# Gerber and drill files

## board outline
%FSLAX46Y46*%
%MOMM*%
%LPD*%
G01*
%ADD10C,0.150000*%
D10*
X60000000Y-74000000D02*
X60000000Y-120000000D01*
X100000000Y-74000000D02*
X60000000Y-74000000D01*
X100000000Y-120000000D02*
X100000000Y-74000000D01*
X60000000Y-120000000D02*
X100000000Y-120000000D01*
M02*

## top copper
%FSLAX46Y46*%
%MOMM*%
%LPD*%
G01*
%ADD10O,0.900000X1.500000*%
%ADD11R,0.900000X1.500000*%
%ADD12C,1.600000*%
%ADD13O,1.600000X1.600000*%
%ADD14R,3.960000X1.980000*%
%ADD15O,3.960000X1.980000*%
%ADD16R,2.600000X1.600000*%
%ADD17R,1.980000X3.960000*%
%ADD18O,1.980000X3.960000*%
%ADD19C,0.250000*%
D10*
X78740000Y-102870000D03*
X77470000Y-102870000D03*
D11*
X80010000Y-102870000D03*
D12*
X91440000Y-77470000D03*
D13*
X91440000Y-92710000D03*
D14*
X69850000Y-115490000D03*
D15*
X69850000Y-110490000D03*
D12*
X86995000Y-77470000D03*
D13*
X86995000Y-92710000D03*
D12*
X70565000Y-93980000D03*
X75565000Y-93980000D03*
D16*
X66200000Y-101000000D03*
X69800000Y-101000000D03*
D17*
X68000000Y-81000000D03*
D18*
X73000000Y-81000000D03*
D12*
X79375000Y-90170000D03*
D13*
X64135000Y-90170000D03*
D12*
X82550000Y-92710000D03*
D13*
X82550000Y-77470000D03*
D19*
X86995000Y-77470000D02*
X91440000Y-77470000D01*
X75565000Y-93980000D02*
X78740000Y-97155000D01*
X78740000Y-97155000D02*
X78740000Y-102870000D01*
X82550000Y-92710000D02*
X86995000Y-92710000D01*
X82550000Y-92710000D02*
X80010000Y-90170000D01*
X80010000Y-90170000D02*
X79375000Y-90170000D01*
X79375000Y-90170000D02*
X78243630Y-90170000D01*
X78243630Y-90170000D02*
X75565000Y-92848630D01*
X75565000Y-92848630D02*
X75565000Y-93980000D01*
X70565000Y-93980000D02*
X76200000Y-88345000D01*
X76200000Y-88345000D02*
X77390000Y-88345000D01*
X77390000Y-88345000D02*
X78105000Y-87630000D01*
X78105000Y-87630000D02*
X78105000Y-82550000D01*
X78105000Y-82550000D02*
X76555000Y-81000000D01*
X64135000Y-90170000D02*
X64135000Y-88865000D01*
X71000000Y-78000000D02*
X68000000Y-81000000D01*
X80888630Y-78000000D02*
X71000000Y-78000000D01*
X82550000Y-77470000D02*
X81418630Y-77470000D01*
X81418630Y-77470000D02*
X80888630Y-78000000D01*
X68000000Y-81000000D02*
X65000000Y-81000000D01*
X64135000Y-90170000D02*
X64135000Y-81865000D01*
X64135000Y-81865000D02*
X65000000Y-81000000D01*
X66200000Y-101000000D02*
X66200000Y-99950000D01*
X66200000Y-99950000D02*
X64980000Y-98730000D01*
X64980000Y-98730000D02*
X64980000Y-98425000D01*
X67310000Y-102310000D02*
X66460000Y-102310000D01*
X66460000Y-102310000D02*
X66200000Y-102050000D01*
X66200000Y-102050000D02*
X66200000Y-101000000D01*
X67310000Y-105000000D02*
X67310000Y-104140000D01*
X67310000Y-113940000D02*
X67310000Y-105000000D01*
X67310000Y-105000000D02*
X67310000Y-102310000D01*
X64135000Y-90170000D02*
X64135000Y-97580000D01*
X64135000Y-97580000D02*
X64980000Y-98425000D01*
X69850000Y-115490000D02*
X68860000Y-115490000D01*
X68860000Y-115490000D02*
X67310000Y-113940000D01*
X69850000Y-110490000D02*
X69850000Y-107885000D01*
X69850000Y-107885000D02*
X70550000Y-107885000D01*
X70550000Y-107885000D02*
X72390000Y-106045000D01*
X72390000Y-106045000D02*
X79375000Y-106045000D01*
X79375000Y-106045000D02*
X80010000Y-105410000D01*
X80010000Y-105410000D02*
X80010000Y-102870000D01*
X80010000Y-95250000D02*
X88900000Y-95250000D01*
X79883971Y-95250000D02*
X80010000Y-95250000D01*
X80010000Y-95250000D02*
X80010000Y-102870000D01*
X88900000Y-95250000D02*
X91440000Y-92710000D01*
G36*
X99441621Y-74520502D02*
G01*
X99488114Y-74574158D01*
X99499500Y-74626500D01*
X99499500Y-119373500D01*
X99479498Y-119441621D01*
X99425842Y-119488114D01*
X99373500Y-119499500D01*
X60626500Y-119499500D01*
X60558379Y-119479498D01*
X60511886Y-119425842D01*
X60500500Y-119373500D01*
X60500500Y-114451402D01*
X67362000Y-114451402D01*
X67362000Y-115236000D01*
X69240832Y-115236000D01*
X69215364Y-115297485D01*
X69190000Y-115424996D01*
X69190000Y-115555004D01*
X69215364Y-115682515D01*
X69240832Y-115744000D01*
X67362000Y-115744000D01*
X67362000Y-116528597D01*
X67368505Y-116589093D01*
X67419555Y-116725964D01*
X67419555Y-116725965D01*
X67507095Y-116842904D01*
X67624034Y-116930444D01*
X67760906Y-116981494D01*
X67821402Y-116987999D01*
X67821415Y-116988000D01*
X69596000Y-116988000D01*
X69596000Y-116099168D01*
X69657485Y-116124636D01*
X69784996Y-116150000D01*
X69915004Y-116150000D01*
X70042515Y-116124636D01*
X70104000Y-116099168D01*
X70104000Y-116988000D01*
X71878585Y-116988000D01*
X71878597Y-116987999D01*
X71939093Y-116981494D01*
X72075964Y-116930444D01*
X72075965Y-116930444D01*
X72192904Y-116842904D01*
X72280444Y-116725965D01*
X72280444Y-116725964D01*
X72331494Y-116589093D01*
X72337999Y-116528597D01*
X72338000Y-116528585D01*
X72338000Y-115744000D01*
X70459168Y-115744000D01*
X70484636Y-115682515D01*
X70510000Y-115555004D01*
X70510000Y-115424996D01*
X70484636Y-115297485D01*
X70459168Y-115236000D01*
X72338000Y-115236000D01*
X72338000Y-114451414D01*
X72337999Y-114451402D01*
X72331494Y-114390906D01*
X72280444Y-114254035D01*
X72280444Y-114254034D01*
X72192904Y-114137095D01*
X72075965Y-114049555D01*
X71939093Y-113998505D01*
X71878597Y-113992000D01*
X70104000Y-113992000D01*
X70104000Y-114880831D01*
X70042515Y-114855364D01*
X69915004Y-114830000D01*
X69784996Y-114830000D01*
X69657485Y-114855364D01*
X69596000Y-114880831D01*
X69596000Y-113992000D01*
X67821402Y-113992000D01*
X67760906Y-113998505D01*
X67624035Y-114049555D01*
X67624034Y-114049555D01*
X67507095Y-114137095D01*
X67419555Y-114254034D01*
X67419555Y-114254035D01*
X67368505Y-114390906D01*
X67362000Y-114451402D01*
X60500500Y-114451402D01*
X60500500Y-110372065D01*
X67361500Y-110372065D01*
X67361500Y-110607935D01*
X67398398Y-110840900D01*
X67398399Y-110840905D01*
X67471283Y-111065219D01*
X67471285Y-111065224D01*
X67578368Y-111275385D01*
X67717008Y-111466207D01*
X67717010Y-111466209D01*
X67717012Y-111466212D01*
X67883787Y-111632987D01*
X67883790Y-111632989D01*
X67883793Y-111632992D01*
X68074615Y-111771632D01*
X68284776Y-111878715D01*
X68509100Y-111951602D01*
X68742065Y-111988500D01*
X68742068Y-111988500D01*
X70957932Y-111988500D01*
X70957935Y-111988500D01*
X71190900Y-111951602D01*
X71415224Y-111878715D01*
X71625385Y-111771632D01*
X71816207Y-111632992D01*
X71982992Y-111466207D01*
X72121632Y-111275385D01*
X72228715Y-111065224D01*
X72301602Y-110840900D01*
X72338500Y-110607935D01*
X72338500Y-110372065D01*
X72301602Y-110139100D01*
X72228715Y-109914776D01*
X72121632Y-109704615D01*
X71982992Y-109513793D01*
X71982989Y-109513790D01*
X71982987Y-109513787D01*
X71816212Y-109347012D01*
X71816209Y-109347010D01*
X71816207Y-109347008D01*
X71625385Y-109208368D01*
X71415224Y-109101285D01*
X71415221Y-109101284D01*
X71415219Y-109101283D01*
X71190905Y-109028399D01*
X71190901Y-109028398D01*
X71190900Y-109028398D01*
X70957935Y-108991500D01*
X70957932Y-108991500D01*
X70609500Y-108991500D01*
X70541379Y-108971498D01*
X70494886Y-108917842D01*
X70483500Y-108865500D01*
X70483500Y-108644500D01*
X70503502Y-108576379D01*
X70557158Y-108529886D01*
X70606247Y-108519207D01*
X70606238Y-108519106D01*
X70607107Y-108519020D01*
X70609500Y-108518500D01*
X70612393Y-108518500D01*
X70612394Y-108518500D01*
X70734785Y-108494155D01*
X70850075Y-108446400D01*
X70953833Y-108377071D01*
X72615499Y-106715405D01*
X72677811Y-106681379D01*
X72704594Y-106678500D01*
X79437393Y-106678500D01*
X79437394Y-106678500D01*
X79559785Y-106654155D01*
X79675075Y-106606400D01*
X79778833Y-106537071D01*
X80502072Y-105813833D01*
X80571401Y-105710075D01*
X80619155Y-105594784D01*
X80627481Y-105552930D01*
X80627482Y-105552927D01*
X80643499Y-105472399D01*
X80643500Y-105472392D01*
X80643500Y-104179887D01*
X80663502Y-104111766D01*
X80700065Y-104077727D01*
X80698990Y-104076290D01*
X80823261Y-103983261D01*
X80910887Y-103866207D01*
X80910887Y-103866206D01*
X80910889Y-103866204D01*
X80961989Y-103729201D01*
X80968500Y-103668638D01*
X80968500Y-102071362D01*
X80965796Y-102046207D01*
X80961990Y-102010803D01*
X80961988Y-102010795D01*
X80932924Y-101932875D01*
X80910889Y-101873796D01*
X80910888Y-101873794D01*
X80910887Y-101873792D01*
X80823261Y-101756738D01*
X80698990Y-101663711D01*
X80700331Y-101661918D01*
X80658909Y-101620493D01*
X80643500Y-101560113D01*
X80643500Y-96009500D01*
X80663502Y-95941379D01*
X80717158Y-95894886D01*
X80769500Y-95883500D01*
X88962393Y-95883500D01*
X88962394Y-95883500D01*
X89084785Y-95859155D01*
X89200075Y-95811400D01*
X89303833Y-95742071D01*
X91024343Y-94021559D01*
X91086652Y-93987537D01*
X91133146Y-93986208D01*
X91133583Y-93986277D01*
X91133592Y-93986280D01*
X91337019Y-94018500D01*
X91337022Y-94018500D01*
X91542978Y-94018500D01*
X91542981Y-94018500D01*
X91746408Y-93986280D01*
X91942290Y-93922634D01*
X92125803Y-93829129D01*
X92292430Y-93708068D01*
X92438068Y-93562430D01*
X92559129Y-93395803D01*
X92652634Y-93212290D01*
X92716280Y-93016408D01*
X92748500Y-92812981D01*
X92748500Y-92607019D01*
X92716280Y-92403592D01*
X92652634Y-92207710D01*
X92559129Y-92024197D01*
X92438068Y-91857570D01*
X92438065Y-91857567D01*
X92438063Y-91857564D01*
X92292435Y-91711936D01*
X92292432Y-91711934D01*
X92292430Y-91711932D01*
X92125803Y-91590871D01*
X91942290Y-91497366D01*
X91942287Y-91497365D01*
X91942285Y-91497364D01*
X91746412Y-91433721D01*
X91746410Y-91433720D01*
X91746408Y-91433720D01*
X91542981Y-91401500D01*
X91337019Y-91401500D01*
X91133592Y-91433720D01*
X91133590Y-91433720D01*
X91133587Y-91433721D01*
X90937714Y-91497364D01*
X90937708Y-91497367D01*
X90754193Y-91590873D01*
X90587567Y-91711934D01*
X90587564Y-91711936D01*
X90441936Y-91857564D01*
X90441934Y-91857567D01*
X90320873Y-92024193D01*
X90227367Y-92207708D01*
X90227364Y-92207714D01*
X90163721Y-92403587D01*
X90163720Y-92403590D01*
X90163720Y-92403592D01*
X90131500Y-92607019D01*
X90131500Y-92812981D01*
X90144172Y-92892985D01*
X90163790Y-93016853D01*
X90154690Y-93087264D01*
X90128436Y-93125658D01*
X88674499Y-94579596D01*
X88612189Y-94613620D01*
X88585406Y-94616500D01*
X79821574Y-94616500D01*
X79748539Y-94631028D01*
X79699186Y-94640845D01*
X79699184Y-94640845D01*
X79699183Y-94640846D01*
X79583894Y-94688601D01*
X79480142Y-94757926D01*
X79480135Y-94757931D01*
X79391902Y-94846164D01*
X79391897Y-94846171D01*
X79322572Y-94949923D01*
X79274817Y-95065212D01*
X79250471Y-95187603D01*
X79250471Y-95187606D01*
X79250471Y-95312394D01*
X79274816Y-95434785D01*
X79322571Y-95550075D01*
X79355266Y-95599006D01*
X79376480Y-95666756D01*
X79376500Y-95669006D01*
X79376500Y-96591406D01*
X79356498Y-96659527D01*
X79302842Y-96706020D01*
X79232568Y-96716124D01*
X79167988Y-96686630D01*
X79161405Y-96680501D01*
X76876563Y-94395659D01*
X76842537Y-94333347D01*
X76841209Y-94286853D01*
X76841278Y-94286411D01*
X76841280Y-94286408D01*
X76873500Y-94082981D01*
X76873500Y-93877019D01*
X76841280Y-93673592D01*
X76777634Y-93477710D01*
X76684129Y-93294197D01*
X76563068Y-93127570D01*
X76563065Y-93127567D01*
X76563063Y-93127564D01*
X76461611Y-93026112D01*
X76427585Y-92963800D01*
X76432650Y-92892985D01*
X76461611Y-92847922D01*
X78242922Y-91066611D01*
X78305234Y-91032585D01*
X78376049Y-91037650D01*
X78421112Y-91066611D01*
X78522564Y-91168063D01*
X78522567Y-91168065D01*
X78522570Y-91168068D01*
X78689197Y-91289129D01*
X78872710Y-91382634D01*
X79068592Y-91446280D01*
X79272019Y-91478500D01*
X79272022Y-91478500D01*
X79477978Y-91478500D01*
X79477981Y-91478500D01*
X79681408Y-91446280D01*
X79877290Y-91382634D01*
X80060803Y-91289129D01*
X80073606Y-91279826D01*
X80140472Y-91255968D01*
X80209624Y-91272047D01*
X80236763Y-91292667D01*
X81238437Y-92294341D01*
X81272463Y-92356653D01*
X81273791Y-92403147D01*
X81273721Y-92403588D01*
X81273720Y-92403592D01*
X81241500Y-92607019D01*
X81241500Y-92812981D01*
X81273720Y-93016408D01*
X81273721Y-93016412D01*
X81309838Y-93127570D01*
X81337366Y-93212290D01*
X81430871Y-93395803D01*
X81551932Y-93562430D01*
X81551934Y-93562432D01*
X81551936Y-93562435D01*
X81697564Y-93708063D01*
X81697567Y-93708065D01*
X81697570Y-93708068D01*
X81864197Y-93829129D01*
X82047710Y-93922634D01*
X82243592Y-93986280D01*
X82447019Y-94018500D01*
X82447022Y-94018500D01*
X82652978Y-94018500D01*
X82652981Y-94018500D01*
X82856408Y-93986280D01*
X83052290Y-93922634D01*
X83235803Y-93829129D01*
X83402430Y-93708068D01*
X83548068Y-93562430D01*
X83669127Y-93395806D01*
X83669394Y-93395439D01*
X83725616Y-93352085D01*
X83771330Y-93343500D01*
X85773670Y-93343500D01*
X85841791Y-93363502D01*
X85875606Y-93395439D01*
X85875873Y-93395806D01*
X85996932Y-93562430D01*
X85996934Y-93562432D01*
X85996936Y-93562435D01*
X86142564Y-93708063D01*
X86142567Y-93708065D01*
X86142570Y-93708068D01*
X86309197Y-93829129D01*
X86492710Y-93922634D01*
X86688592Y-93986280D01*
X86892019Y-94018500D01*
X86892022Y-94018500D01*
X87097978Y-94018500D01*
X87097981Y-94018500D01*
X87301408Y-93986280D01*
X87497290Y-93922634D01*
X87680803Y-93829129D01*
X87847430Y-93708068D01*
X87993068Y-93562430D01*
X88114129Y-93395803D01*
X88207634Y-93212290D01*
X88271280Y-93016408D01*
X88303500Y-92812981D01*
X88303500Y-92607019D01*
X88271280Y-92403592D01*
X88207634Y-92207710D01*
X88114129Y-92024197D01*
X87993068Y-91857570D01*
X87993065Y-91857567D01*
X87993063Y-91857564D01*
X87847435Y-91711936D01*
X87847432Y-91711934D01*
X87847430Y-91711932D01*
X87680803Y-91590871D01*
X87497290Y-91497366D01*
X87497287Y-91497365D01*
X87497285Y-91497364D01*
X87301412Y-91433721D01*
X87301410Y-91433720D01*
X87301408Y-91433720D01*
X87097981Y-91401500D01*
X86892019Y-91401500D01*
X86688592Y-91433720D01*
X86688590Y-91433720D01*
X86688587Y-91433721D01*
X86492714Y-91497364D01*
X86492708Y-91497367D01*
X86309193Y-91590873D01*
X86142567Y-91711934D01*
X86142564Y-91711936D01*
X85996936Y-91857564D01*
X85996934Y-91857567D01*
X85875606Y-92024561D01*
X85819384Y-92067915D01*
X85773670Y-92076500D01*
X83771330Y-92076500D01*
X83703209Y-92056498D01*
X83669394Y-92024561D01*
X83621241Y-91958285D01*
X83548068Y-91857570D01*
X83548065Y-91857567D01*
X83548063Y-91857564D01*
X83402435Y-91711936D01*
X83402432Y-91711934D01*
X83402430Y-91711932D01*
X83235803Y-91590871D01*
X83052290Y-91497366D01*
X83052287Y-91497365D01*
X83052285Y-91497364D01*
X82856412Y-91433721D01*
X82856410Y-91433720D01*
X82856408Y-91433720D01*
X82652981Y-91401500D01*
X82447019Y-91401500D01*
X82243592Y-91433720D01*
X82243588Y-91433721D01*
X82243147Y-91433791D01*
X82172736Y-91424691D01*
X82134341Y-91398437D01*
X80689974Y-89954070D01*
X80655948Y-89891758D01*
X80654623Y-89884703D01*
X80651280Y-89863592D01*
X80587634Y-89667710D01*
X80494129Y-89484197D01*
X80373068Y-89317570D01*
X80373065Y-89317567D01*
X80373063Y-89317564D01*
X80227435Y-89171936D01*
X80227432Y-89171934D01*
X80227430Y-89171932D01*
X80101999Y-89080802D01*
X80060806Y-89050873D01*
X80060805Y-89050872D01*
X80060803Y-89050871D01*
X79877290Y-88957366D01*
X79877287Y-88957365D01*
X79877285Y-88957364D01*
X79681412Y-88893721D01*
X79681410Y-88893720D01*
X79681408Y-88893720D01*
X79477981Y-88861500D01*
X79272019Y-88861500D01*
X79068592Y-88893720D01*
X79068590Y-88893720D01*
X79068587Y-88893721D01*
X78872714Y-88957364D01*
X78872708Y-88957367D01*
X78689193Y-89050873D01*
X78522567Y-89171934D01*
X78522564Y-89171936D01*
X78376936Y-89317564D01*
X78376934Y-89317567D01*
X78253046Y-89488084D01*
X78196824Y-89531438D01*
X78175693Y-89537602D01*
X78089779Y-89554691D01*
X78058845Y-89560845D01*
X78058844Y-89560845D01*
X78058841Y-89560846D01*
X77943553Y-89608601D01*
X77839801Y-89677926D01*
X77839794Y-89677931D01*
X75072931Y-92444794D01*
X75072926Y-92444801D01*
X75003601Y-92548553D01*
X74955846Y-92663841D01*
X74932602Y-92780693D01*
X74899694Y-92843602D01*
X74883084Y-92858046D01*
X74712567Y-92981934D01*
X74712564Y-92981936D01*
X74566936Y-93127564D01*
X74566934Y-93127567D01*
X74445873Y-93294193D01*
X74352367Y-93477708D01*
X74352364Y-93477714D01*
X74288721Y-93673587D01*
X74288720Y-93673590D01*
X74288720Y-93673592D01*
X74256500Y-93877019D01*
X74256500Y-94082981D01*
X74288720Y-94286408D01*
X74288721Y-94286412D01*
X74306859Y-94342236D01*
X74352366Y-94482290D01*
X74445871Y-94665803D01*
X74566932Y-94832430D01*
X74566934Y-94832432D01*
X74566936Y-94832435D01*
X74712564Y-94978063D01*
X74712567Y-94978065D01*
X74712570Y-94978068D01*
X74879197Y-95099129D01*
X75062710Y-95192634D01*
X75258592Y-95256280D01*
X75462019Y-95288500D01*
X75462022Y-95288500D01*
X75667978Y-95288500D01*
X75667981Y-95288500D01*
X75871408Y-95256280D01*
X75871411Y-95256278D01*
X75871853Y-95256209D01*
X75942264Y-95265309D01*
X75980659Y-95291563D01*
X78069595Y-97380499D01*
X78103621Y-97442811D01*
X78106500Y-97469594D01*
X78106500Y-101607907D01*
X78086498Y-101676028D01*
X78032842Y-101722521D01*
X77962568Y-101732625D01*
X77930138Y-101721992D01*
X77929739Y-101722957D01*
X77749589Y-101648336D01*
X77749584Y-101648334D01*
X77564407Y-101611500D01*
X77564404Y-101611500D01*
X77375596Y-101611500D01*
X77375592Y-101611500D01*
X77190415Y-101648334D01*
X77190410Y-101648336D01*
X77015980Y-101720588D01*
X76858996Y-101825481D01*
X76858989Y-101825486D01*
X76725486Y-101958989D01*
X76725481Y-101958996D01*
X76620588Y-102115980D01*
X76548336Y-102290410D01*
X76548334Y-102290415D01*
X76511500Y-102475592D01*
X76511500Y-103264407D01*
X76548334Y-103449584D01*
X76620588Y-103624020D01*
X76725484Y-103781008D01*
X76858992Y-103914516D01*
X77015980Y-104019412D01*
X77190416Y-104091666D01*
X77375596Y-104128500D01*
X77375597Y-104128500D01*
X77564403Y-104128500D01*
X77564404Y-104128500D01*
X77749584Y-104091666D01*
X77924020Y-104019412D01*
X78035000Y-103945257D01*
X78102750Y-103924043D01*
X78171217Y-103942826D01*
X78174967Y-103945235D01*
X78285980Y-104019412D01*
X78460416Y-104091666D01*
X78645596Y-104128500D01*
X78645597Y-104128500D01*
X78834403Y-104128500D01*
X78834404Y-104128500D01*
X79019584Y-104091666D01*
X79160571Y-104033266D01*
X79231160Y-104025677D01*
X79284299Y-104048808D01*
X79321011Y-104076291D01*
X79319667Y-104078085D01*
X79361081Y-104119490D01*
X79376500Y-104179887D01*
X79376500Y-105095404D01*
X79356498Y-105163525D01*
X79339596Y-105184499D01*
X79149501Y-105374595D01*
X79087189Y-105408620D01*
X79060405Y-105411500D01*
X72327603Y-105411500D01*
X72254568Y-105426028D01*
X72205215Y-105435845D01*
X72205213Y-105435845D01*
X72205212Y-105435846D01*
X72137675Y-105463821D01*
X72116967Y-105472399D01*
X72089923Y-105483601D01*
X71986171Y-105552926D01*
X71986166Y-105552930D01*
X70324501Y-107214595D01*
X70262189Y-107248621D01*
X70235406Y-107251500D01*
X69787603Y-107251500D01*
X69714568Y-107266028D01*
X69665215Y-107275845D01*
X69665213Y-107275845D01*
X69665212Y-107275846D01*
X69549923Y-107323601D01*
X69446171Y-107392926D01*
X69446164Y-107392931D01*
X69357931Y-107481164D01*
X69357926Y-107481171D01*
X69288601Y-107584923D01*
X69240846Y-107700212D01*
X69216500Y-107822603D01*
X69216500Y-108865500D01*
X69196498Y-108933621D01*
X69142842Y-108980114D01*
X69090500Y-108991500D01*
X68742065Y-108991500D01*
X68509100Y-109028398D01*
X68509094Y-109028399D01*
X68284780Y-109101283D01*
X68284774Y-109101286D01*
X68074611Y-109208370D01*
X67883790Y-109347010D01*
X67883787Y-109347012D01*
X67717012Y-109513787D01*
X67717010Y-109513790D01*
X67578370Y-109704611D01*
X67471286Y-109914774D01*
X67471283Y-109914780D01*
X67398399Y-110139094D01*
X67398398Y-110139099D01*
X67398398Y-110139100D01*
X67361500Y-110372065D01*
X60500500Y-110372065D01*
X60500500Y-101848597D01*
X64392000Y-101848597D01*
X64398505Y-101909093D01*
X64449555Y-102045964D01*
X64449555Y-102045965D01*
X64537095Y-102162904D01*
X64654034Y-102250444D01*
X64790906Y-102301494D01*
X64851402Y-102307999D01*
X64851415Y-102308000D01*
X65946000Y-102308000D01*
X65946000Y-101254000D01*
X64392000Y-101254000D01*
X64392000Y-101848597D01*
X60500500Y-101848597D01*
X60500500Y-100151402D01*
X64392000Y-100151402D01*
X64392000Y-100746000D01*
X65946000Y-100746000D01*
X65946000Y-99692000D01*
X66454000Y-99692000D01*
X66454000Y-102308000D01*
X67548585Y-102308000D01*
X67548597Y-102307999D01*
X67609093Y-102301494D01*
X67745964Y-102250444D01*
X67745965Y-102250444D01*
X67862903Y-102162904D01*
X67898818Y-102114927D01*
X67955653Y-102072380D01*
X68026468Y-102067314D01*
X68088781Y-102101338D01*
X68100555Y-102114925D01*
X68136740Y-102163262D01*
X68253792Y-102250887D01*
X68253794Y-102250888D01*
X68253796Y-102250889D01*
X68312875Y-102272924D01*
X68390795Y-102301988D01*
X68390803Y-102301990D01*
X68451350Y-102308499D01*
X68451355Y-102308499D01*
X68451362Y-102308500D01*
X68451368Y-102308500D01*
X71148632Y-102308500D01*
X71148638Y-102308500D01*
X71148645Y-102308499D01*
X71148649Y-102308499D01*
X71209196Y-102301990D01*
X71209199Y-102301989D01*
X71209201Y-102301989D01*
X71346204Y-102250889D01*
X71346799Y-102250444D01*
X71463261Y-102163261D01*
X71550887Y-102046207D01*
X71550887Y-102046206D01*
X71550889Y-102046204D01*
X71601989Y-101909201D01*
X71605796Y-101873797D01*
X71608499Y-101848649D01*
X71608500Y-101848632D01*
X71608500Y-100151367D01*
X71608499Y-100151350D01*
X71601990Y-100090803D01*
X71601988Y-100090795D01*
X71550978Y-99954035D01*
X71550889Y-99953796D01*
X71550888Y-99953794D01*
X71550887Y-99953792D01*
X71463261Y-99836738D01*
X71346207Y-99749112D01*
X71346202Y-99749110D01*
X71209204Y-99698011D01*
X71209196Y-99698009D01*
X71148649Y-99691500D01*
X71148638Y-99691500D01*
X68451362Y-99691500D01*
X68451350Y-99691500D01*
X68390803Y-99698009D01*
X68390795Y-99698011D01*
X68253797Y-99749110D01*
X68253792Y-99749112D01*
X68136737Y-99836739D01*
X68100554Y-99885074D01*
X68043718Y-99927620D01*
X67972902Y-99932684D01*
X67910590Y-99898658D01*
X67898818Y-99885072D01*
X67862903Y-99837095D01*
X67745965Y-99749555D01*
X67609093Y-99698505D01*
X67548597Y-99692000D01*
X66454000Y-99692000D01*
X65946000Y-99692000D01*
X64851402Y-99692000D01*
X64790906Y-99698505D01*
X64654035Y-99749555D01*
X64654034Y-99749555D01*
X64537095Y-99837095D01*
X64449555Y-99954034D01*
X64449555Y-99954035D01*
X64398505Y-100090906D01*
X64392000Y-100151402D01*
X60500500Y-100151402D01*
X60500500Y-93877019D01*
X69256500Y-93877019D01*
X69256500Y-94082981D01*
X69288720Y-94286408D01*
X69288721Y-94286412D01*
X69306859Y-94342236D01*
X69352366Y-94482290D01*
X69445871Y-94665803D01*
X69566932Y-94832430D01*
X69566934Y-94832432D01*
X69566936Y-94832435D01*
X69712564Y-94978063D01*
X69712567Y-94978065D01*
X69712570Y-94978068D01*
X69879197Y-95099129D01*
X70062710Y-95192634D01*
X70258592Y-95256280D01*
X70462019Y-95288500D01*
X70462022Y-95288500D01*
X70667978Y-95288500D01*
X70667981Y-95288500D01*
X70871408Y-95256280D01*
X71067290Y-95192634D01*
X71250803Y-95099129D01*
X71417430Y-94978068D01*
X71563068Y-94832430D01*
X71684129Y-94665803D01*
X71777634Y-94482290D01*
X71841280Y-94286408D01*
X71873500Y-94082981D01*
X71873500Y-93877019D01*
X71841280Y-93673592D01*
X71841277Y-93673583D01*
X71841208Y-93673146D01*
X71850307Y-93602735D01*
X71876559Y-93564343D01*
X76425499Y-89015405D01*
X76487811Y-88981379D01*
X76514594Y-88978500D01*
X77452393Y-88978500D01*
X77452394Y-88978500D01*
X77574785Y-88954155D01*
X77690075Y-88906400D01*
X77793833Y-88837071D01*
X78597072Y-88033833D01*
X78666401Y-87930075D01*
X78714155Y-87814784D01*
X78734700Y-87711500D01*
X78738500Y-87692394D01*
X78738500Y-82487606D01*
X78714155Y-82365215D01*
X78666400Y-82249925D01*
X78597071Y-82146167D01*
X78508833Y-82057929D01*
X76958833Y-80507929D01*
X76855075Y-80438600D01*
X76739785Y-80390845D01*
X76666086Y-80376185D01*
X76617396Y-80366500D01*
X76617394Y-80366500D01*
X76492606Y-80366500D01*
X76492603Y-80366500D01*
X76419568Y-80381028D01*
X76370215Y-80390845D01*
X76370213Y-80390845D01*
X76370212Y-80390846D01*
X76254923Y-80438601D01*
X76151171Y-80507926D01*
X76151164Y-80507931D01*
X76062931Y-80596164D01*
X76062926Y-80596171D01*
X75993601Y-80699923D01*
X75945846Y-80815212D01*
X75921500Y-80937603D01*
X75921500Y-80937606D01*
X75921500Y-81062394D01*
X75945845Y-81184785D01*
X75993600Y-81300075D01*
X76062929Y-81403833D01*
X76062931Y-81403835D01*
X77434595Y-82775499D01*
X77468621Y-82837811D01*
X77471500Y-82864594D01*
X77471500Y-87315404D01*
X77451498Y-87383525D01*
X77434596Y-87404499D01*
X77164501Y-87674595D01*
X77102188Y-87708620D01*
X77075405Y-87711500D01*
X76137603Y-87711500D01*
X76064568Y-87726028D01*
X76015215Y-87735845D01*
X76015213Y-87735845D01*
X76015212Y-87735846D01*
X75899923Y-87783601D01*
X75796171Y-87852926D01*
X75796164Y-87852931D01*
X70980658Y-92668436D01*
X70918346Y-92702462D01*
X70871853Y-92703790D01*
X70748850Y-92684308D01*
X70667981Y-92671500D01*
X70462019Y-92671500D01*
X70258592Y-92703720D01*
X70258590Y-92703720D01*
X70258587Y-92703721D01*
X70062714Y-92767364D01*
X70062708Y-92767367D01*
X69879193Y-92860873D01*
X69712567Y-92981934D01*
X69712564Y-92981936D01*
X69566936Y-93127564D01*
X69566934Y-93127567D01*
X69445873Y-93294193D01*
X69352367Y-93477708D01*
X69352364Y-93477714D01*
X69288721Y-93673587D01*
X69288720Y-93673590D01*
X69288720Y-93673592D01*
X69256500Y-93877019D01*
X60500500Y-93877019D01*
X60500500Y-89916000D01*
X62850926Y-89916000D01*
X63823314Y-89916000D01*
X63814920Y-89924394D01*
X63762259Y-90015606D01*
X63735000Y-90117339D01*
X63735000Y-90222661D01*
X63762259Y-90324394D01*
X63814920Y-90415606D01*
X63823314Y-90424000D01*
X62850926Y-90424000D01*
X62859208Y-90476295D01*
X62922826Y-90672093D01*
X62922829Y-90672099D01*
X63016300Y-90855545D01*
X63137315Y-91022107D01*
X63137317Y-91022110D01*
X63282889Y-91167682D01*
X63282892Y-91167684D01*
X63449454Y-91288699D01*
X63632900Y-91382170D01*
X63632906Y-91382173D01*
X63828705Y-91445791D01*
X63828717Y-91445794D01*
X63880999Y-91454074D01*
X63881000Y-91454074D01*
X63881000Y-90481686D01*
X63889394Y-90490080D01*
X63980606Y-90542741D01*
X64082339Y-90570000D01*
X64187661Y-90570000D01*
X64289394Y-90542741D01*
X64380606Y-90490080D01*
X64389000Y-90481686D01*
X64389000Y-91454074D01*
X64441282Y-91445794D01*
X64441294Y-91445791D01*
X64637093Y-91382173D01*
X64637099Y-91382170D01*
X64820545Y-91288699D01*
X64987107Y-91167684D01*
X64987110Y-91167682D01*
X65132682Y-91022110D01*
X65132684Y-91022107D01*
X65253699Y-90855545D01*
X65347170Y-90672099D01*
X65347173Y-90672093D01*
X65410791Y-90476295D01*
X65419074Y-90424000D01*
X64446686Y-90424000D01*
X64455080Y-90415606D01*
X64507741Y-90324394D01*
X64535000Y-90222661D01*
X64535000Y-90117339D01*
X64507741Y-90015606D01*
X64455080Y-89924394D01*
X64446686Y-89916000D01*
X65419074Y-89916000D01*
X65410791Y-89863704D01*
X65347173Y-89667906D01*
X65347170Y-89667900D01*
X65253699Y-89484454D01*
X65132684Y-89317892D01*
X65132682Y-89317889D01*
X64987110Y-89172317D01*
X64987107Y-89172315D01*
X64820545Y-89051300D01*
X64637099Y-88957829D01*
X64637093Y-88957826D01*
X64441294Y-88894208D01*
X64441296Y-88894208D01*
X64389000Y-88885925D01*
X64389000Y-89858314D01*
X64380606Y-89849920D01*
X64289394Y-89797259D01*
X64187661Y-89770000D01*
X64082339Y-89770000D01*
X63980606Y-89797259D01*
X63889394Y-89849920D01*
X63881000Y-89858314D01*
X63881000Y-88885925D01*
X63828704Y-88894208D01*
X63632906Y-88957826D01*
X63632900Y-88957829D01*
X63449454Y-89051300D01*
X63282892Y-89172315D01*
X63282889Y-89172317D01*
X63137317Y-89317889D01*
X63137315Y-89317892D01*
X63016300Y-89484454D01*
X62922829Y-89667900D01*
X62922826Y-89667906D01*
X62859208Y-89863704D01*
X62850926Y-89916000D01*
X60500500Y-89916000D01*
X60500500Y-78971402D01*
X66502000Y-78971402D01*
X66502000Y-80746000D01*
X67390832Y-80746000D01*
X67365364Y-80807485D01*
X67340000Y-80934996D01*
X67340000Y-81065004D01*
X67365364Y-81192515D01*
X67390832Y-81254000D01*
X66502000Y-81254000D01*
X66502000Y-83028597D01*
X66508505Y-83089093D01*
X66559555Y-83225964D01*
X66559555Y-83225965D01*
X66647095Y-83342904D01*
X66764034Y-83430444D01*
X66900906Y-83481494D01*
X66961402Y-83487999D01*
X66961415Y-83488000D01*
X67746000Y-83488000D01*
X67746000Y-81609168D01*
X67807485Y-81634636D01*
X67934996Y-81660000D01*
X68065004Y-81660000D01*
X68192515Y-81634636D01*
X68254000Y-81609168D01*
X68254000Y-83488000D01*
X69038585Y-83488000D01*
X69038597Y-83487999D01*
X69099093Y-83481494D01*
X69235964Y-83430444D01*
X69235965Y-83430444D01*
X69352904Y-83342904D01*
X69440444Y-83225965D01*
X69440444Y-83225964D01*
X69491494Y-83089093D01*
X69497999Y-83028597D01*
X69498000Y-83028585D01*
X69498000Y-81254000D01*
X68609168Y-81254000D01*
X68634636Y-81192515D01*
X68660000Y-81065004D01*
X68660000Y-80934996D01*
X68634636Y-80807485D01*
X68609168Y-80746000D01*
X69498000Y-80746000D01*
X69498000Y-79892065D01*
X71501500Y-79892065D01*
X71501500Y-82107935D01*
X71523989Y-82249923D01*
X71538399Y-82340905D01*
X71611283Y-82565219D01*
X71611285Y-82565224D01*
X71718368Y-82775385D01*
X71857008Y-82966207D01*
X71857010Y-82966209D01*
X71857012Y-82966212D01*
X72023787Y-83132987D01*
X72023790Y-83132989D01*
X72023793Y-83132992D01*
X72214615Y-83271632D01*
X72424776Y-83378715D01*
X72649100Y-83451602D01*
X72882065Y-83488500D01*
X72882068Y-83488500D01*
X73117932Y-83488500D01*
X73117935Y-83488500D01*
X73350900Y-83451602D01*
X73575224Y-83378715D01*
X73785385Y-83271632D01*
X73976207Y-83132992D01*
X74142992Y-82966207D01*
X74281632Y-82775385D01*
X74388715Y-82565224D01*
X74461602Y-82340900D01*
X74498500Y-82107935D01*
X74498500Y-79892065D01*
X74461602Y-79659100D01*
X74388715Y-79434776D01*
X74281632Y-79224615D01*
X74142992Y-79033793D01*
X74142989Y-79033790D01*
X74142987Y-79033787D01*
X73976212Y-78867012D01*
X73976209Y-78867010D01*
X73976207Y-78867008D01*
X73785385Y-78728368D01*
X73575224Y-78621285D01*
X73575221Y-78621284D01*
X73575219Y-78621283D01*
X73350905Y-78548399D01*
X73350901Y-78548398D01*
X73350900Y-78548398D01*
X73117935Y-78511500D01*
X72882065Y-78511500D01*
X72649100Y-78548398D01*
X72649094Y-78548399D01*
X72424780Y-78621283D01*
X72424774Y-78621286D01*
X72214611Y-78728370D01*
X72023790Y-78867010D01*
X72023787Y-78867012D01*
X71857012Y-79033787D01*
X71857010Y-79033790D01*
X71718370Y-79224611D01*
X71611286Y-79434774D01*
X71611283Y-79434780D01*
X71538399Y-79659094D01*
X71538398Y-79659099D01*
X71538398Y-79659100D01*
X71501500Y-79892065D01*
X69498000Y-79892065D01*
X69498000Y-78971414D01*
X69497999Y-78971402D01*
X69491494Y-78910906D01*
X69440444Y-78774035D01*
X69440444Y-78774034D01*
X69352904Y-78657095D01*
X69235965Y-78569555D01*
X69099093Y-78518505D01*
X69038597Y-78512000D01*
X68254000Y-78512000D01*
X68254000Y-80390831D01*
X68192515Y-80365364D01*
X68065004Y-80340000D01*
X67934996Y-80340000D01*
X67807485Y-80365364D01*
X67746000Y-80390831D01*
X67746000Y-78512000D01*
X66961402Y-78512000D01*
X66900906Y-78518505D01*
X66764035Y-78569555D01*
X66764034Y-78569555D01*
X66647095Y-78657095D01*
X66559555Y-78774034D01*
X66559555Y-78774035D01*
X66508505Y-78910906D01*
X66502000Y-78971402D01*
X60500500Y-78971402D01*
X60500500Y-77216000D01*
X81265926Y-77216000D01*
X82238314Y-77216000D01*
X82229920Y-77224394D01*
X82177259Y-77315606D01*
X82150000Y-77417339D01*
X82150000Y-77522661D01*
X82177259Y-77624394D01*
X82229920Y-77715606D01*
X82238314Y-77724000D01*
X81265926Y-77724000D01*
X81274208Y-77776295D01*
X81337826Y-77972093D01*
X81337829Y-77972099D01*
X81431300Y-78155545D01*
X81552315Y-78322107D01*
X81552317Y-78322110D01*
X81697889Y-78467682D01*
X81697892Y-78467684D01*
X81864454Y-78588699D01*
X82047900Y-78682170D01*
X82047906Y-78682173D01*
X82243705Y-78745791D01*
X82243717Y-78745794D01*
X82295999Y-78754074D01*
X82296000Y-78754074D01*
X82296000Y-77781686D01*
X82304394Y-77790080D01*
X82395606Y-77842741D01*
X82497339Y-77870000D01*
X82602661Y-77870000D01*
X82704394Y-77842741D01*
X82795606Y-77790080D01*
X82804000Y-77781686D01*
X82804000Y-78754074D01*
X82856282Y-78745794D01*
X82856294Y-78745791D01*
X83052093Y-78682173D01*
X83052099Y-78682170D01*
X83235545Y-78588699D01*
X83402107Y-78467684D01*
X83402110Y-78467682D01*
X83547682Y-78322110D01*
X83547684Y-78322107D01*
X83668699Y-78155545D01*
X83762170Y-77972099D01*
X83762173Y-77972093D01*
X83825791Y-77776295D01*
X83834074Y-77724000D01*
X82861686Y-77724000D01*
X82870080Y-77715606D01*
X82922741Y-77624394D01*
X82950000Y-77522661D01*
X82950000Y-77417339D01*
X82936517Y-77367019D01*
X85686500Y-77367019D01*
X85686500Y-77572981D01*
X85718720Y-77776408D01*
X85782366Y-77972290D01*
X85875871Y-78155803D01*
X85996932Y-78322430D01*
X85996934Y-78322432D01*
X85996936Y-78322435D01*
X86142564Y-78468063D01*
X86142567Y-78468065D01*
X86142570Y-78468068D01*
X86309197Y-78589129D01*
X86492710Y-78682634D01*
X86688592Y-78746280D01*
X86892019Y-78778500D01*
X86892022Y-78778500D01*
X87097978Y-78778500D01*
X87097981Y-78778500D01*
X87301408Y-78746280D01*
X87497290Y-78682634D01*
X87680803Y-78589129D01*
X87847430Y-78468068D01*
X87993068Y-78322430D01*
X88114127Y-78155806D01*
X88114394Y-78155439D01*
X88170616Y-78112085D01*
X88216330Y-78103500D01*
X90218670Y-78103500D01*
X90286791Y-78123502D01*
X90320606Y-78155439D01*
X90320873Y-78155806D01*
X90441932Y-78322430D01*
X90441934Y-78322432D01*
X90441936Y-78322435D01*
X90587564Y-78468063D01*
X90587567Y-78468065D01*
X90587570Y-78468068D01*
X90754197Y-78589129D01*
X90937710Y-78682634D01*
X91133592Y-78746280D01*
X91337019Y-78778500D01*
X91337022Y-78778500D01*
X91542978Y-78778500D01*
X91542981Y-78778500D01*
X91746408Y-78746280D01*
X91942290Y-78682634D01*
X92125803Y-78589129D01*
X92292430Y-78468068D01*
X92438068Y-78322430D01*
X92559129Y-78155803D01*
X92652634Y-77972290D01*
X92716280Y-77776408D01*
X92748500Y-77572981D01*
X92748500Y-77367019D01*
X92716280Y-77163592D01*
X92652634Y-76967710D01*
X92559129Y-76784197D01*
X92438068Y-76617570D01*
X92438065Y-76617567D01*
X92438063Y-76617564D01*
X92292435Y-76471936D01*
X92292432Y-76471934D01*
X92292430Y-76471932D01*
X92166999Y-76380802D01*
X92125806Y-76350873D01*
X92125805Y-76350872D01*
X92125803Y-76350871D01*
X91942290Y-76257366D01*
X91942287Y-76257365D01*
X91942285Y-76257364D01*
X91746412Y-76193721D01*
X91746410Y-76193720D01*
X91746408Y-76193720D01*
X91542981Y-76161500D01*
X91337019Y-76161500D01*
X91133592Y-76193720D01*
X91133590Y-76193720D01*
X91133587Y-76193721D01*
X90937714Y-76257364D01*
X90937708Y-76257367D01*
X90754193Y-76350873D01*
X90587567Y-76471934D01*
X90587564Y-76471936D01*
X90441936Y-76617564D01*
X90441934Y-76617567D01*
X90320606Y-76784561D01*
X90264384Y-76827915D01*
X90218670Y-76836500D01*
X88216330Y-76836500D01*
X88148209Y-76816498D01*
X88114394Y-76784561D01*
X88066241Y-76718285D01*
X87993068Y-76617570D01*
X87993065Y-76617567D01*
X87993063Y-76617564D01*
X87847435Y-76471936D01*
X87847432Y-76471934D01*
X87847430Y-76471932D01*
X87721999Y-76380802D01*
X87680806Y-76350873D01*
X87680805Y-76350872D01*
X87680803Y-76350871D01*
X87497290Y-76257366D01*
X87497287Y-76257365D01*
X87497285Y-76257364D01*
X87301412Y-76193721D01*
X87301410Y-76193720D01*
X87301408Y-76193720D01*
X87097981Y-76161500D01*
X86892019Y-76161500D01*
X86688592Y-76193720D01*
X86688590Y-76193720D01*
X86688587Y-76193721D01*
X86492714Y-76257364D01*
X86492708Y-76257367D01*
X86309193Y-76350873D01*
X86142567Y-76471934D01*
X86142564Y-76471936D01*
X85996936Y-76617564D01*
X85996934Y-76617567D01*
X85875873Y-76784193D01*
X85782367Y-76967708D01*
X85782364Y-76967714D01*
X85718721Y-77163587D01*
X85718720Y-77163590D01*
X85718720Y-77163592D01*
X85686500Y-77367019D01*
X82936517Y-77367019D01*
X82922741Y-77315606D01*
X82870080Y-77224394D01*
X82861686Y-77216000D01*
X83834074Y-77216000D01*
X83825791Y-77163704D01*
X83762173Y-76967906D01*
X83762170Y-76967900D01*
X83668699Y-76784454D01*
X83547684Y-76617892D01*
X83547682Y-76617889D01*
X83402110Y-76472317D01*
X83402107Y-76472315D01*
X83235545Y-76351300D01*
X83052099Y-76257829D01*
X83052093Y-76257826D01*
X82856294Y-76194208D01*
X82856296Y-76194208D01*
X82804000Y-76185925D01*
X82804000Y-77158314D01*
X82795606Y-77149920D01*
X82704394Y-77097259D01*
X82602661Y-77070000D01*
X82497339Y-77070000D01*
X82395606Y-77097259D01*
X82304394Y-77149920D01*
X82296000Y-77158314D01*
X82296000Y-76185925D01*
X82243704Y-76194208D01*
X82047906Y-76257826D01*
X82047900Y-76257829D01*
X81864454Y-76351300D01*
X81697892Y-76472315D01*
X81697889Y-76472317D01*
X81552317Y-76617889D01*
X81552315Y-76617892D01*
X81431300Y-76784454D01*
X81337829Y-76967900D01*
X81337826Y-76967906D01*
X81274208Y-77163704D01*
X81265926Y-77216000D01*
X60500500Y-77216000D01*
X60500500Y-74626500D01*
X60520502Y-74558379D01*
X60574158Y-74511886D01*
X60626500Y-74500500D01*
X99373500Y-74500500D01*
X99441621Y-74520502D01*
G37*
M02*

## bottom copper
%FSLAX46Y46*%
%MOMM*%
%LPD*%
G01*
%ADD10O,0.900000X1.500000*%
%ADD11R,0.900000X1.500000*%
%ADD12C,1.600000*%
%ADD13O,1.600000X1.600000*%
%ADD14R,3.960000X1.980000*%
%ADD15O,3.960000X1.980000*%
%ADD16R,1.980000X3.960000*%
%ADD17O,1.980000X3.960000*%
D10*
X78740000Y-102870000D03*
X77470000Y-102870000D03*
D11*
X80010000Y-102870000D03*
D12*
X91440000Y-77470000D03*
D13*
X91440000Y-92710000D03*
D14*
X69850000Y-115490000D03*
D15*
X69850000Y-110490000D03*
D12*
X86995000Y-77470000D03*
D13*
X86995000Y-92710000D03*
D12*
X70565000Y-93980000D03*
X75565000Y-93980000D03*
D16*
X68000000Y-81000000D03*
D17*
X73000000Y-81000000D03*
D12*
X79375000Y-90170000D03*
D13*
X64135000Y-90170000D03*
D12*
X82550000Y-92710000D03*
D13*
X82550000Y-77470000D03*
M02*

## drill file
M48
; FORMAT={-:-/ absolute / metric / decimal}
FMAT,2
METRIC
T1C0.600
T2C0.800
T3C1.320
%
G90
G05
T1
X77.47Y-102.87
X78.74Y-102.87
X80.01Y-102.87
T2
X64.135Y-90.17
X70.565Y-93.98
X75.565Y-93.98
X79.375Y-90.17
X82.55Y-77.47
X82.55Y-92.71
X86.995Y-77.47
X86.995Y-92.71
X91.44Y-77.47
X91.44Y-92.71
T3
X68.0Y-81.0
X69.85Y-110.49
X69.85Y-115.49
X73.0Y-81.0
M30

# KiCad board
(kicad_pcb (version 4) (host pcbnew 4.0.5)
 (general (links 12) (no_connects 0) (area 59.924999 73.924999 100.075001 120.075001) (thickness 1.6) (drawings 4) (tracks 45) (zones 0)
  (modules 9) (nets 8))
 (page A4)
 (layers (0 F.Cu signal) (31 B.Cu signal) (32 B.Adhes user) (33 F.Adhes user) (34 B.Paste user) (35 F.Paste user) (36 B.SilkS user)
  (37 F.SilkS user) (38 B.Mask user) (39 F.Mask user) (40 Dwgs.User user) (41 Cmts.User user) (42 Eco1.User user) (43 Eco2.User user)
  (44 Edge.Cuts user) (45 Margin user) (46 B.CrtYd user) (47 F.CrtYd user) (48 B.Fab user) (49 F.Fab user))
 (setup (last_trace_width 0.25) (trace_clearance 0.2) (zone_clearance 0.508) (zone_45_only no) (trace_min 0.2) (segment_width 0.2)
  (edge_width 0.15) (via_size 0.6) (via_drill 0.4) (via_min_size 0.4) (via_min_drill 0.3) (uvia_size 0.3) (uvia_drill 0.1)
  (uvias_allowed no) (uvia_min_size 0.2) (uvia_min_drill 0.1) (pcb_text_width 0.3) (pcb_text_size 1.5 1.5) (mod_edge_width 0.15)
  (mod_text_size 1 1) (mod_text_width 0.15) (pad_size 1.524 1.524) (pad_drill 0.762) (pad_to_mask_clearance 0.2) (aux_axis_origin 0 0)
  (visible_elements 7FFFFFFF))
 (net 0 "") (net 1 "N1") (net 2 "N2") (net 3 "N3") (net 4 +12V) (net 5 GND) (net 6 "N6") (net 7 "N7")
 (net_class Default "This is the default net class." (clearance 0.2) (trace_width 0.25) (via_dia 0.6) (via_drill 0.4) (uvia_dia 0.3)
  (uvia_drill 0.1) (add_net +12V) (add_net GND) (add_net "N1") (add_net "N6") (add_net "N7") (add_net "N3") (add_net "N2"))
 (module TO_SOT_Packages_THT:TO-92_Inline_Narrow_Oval (layer F.Cu) (at 80.01 102.87 180)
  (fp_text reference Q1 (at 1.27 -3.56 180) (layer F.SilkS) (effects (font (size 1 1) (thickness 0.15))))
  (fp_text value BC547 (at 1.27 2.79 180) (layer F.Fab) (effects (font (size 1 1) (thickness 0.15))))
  (pad 2 thru_hole oval (at 1.27 0) (size 0.9 1.5) (drill 0.6) (layers *.Cu *.Mask) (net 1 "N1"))
  (pad 3 thru_hole oval (at 2.54 0) (size 0.9 1.5) (drill 0.6) (layers *.Cu *.Mask) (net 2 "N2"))
  (pad 1 thru_hole rect (at 0 0) (size 0.9 1.5) (drill 0.6) (layers *.Cu *.Mask) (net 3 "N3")))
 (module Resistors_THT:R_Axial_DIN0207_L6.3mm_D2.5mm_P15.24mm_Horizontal (layer F.Cu) (at 91.44 77.47 270)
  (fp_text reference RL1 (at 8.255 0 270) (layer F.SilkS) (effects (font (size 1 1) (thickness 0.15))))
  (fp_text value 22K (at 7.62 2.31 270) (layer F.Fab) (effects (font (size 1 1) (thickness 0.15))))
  (pad 1 thru_hole circle (at 0 0 270) (size 1.6 1.6) (drill 0.8) (layers *.Cu *.Mask) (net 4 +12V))
  (pad 2 thru_hole oval (at 15.24 0 270) (size 1.6 1.6) (drill 0.8) (layers *.Cu *.Mask) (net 3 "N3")))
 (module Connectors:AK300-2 (layer F.Cu) (at 69.85 115.49 90)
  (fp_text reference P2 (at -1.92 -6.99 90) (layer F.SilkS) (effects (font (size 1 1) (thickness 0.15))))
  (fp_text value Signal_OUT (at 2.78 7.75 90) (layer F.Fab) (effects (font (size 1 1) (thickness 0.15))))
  (pad 1 thru_hole rect (at 0 0 90) (size 1.98 3.96) (drill 1.32) (layers *.Cu F.Paste F.Mask) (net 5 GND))
  (pad 2 thru_hole oval (at 5 0 90) (size 1.98 3.96) (drill 1.32) (layers *.Cu F.Paste F.Mask) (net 3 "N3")))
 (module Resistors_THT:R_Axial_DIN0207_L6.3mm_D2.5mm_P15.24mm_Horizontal (layer F.Cu) (at 86.995 77.47 270)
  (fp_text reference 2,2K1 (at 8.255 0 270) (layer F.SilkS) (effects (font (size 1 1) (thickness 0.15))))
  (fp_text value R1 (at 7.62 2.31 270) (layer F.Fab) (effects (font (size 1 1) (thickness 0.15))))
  (pad 1 thru_hole circle (at 0 0 270) (size 1.6 1.6) (drill 0.8) (layers *.Cu *.Mask) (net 4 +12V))
  (pad 2 thru_hole oval (at 15.24 0 270) (size 1.6 1.6) (drill 0.8) (layers *.Cu *.Mask) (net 1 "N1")))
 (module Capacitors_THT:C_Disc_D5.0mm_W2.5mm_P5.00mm (layer F.Cu) (at 70.565 93.98)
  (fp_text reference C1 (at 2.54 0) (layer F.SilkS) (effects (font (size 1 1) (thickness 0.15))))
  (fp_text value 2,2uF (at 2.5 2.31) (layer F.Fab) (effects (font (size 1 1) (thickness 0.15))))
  (pad 1 thru_hole circle (at 0 0) (size 1.6 1.6) (drill 0.8) (layers *.Cu *.Mask) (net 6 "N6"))
  (pad 2 thru_hole circle (at 5 0) (size 1.6 1.6) (drill 0.8) (layers *.Cu *.Mask) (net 1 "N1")))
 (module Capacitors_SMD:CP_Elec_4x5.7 (layer F.Cu) (at 68 101)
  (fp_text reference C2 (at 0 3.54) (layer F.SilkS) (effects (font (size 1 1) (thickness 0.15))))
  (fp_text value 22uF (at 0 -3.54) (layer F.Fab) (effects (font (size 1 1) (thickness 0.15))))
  (pad 1 smd rect (at -1.8 0 180) (size 2.6 1.6) (layers F.Cu F.Paste F.Mask) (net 5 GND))
  (pad 2 smd rect (at 1.8 0 180) (size 2.6 1.6) (layers F.Cu F.Paste F.Mask) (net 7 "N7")))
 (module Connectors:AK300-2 (layer F.Cu) (at 68 81)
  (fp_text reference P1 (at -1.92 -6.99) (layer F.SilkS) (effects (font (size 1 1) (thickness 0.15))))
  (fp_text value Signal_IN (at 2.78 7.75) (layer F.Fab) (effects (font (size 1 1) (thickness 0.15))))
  (pad 1 thru_hole rect (at 0 0) (size 1.98 3.96) (drill 1.32) (layers *.Cu F.Paste F.Mask) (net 5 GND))
  (pad 2 thru_hole oval (at 5 0) (size 1.98 3.96) (drill 1.32) (layers *.Cu F.Paste F.Mask) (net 6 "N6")))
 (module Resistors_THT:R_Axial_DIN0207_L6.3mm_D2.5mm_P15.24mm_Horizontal (layer F.Cu) (at 79.375 90.17 180)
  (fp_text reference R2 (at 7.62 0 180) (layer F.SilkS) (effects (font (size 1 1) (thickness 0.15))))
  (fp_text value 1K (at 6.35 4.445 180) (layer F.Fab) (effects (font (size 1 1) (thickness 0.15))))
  (pad 1 thru_hole circle (at 0 0 180) (size 1.6 1.6) (drill 0.8) (layers *.Cu *.Mask) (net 1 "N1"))
  (pad 2 thru_hole oval (at 15.24 0 180) (size 1.6 1.6) (drill 0.8) (layers *.Cu *.Mask) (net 5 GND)))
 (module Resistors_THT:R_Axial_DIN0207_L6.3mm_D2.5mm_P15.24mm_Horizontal (layer F.Cu) (at 82.55 92.71 90)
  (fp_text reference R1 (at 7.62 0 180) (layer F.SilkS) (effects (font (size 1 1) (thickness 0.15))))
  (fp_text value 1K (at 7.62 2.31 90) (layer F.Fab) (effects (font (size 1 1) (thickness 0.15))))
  (pad 1 thru_hole circle (at 0 0 90) (size 1.6 1.6) (drill 0.8) (layers *.Cu *.Mask) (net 1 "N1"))
  (pad 2 thru_hole oval (at 15.24 0 90) (size 1.6 1.6) (drill 0.8) (layers *.Cu *.Mask) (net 5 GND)))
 (gr_line (start 60 74) (end 60 120) (layer Edge.Cuts) (width 0.15))
 (gr_line (start 100 74) (end 60 74) (layer Edge.Cuts) (width 0.15))
 (gr_line (start 100 120) (end 100 74) (layer Edge.Cuts) (width 0.15))
 (gr_line (start 60 120) (end 100 120) (layer Edge.Cuts) (width 0.15))
 (segment (start 86.995 77.47) (end 91.44 77.47) (width 0.25) (layer F.Cu) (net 4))
 (segment (start 75.565 93.98) (end 78.74 97.155) (width 0.25) (layer F.Cu) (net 1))
 (segment (start 78.74 97.155) (end 78.74 102.87) (width 0.25) (layer F.Cu) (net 1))
 (segment (start 82.55 92.71) (end 86.995 92.71) (width 0.25) (layer F.Cu) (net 1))
 (segment (start 82.55 92.71) (end 80.01 90.17) (width 0.25) (layer F.Cu) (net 1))
 (segment (start 80.01 90.17) (end 79.375 90.17) (width 0.25) (layer F.Cu) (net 1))
 (segment (start 79.375 90.17) (end 78.24363 90.17) (width 0.25) (layer F.Cu) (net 1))
 (segment (start 78.24363 90.17) (end 75.565 92.84863) (width 0.25) (layer F.Cu) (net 1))
 (segment (start 75.565 92.84863) (end 75.565 93.98) (width 0.25) (layer F.Cu) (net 1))
 (segment (start 70.565 93.98) (end 76.2 88.345) (width 0.25) (layer F.Cu) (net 6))
 (segment (start 76.2 88.345) (end 77.39 88.345) (width 0.25) (layer F.Cu) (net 6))
 (segment (start 77.39 88.345) (end 78.105 87.63) (width 0.25) (layer F.Cu) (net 6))
 (segment (start 78.105 87.63) (end 78.105 82.55) (width 0.25) (layer F.Cu) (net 6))
 (segment (start 78.105 82.55) (end 76.555 81) (width 0.25) (layer F.Cu) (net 6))
 (segment (start 64.135 90.17) (end 64.135 88.865) (width 0.25) (layer F.Cu) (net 5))
 (segment (start 71 78) (end 68 81) (width 0.25) (layer F.Cu) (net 5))
 (segment (start 80.88863 78) (end 71 78) (width 0.25) (layer F.Cu) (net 5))
 (segment (start 82.55 77.47) (end 81.41863 77.47) (width 0.25) (layer F.Cu) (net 5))
 (segment (start 81.41863 77.47) (end 80.88863 78) (width 0.25) (layer F.Cu) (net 5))
 (segment (start 68 81) (end 65 81) (width 0.25) (layer F.Cu) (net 5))
 (segment (start 64.135 90.17) (end 64.135 81.865) (width 0.25) (layer F.Cu) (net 5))
 (segment (start 64.135 81.865) (end 65 81) (width 0.25) (layer F.Cu) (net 5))
 (segment (start 66.2 101) (end 66.2 99.95) (width 0.25) (layer F.Cu) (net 5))
 (segment (start 66.2 99.95) (end 64.98 98.73) (width 0.25) (layer F.Cu) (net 5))
 (segment (start 64.98 98.73) (end 64.98 98.425) (width 0.25) (layer F.Cu) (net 5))
 (segment (start 67.31 102.31) (end 66.46 102.31) (width 0.25) (layer F.Cu) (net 5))
 (segment (start 66.46 102.31) (end 66.2 102.05) (width 0.25) (layer F.Cu) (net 5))
 (segment (start 66.2 102.05) (end 66.2 101) (width 0.25) (layer F.Cu) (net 5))
 (segment (start 67.31 105) (end 67.31 104.14) (width 0.25) (layer F.Cu) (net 5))
 (segment (start 67.31 113.94) (end 67.31 105) (width 0.25) (layer F.Cu) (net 5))
 (segment (start 67.31 105) (end 67.31 102.31) (width 0.25) (layer F.Cu) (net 5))
 (segment (start 64.135 90.17) (end 64.135 97.58) (width 0.25) (layer F.Cu) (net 5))
 (segment (start 64.135 97.58) (end 64.98 98.425) (width 0.25) (layer F.Cu) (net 5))
 (segment (start 69.85 115.49) (end 68.86 115.49) (width 0.25) (layer F.Cu) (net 5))
 (segment (start 68.86 115.49) (end 67.31 113.94) (width 0.25) (layer F.Cu) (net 5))
 (segment (start 69.85 110.49) (end 69.85 107.885) (width 0.25) (layer F.Cu) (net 3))
 (segment (start 69.85 107.885) (end 70.55 107.885) (width 0.25) (layer F.Cu) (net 3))
 (segment (start 70.55 107.885) (end 72.39 106.045) (width 0.25) (layer F.Cu) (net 3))
 (segment (start 72.39 106.045) (end 79.375 106.045) (width 0.25) (layer F.Cu) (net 3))
 (segment (start 79.375 106.045) (end 80.01 105.41) (width 0.25) (layer F.Cu) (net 3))
 (segment (start 80.01 105.41) (end 80.01 102.87) (width 0.25) (layer F.Cu) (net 3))
 (segment (start 80.01 95.25) (end 88.9 95.25) (width 0.25) (layer F.Cu) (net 3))
 (segment (start 79.883971 95.25) (end 80.01 95.25) (width 0.25) (layer F.Cu) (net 3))
 (segment (start 80.01 95.25) (end 80.01 102.87) (width 0.25) (layer F.Cu) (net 3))
 (segment (start 88.9 95.25) (end 91.44 92.71) (width 0.25) (layer F.Cu) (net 3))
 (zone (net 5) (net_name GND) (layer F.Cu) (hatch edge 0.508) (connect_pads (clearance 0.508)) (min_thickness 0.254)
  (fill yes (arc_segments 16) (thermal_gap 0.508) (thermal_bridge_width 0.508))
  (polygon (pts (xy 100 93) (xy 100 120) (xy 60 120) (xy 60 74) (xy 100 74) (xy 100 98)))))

